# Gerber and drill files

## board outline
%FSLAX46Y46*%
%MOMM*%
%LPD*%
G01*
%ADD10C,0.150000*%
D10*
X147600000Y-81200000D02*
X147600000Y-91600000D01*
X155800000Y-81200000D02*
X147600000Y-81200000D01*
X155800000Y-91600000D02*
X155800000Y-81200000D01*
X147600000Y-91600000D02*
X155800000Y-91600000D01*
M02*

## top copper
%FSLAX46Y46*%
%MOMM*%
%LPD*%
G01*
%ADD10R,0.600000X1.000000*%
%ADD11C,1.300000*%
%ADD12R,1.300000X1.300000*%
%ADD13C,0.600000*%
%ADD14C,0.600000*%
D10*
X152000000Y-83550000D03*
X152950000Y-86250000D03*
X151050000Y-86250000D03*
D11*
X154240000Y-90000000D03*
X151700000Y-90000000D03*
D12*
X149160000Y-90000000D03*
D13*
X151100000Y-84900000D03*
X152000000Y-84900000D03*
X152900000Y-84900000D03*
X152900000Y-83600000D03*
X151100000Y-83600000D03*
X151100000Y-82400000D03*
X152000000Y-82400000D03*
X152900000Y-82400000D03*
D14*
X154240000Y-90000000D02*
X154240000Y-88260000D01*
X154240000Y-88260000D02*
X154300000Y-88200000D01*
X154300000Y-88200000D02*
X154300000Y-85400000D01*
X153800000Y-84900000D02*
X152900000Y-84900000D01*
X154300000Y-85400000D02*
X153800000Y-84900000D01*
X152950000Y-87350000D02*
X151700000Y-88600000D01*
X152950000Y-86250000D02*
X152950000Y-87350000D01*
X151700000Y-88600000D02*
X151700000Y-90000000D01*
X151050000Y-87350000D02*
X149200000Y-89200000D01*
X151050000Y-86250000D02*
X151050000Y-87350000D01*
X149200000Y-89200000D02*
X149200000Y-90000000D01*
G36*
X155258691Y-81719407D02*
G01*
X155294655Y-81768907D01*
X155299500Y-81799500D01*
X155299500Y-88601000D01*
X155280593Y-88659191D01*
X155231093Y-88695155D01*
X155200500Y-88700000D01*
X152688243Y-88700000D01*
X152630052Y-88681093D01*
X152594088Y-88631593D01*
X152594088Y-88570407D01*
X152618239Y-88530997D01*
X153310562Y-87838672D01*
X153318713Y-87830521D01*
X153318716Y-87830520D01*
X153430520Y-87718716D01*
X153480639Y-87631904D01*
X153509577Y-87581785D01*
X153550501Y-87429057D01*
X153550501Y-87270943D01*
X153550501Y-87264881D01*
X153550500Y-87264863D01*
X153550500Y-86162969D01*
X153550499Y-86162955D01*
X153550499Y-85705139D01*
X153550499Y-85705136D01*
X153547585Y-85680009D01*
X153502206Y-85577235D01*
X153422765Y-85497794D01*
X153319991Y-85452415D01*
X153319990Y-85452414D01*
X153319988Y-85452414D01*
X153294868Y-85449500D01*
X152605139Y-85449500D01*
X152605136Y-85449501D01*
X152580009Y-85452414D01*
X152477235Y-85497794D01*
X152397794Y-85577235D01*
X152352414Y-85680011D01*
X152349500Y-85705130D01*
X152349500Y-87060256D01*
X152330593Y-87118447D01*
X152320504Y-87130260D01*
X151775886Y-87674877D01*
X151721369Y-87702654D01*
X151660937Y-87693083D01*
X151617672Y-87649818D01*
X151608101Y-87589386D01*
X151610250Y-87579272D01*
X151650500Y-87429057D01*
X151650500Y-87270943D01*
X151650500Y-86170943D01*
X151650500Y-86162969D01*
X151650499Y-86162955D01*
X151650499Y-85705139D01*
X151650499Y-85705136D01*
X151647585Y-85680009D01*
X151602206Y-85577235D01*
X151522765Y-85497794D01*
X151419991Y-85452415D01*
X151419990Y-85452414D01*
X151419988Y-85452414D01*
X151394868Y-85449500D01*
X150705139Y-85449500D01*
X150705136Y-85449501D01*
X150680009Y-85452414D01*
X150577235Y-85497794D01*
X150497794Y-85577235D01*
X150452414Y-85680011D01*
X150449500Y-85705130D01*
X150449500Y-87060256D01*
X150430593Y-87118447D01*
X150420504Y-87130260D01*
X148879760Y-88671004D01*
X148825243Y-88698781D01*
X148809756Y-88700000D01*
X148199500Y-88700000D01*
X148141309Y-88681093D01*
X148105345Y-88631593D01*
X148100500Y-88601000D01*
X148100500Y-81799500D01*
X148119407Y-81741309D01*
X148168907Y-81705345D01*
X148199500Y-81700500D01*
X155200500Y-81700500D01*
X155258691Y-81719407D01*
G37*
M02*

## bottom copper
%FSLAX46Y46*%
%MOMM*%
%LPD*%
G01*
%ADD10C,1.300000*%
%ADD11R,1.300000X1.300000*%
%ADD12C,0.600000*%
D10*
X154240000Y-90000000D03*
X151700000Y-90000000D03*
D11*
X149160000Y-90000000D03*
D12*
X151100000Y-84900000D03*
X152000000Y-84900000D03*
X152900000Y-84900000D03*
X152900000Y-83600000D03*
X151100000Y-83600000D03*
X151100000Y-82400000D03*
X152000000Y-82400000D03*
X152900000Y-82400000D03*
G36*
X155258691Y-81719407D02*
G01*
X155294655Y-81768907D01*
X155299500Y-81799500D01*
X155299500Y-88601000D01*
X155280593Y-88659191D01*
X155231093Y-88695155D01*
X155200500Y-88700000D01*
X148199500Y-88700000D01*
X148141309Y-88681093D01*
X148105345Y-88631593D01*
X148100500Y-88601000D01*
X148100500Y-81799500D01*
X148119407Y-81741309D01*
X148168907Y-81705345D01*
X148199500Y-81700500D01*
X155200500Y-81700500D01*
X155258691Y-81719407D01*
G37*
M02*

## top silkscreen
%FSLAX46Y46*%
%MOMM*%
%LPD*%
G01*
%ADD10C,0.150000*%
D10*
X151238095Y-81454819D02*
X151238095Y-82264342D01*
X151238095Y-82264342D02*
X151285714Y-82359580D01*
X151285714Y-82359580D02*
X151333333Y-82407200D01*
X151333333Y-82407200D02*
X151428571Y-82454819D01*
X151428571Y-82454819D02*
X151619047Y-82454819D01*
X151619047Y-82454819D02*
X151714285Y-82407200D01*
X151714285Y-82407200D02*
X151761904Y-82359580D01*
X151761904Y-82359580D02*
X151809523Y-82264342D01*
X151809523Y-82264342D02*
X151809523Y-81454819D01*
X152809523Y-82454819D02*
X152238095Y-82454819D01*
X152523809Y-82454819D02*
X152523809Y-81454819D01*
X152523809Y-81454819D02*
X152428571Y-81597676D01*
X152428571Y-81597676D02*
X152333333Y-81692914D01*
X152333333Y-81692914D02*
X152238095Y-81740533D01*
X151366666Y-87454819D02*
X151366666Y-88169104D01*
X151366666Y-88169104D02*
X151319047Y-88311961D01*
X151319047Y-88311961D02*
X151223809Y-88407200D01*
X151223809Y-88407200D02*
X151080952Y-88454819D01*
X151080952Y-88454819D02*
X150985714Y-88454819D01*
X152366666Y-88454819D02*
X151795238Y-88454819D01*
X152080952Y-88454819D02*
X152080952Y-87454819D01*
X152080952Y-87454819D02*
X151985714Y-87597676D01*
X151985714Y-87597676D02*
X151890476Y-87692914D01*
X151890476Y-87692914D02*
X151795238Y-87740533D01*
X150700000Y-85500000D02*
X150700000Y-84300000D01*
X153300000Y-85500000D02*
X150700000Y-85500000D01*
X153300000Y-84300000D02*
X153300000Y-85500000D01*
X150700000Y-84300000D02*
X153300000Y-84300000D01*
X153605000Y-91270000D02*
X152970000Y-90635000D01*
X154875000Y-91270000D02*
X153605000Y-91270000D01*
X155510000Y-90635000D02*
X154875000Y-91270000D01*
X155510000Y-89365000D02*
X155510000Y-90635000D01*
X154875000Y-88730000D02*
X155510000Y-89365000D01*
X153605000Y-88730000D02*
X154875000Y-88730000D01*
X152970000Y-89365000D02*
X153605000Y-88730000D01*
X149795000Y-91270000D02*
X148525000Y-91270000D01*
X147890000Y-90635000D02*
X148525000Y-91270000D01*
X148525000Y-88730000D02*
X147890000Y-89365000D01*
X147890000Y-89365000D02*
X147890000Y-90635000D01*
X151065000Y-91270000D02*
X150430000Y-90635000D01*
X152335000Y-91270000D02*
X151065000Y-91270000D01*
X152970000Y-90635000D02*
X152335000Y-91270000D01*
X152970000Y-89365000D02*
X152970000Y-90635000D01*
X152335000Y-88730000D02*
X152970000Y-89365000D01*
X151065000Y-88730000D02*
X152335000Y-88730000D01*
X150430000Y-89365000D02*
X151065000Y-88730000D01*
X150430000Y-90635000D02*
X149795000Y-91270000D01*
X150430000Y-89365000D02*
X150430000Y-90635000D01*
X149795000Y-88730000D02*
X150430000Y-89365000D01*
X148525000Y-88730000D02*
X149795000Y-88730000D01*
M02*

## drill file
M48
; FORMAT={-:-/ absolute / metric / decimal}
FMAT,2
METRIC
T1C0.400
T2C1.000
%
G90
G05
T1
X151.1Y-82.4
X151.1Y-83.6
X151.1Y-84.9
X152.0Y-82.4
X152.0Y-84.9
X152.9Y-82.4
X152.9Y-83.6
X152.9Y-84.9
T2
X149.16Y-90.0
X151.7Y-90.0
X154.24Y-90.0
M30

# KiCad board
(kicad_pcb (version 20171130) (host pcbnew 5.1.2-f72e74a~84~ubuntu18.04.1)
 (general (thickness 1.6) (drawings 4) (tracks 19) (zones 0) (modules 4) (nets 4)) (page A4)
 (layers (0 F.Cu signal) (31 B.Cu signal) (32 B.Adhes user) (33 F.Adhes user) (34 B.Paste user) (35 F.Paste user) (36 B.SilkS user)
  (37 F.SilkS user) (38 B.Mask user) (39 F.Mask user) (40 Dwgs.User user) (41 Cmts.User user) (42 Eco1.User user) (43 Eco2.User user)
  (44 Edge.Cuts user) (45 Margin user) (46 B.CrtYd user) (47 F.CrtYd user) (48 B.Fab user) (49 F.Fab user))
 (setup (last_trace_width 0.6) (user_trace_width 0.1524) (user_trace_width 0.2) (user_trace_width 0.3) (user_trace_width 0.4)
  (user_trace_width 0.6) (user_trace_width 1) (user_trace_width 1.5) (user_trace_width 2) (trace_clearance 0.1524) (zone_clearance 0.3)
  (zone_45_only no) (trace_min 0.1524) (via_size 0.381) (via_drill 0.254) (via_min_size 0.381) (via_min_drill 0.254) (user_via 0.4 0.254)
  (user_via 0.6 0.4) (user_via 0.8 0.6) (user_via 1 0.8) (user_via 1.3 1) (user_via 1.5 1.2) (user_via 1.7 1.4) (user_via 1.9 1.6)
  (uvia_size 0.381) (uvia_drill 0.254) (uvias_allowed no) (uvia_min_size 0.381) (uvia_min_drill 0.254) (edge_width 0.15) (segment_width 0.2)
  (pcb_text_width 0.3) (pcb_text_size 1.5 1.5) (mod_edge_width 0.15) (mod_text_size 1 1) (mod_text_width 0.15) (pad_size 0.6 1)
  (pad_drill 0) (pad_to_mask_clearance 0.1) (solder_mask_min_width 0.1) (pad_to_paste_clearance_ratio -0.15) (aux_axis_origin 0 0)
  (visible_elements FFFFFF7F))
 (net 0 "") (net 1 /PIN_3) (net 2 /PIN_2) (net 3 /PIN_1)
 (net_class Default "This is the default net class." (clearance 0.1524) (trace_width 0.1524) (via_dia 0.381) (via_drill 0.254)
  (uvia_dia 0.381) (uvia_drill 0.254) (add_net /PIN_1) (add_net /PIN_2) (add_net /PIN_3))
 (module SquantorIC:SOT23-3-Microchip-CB (layer F.Cu) (at 152 84.9)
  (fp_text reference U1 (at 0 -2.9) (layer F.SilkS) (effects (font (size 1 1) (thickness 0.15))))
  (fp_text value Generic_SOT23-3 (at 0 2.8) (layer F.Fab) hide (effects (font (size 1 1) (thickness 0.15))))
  (fp_line (start -1.3 0.6) (end -1.3 -0.6) (layer F.SilkS) (width 0.15))
  (fp_line (start 1.3 0.6) (end -1.3 0.6) (layer F.SilkS) (width 0.15))
  (fp_line (start 1.3 -0.6) (end 1.3 0.6) (layer F.SilkS) (width 0.15))
  (fp_line (start -1.3 -0.6) (end 1.3 -0.6) (layer F.SilkS) (width 0.15))
  (pad 3 smd rect (at 0 -1.35) (size 0.6 1) (layers F.Cu F.Paste F.Mask) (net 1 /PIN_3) (zone_connect 2))
  (pad 2 smd rect (at 0.95 1.35) (size 0.6 1) (layers F.Cu F.Paste F.Mask) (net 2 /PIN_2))
  (pad 1 smd rect (at -0.95 1.35) (size 0.6 1) (layers F.Cu F.Paste F.Mask) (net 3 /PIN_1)))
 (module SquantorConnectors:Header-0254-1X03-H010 (layer F.Cu) (at 151.7 90)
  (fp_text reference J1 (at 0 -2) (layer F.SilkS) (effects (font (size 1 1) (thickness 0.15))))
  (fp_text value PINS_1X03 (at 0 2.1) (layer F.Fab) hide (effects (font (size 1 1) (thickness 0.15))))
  (fp_line (start 1.905 1.27) (end 1.27 0.635) (layer F.SilkS) (width 0.15))
  (fp_line (start 3.175 1.27) (end 1.905 1.27) (layer F.SilkS) (width 0.15))
  (fp_line (start 3.81 0.635) (end 3.175 1.27) (layer F.SilkS) (width 0.15))
  (fp_line (start 3.81 -0.635) (end 3.81 0.635) (layer F.SilkS) (width 0.15))
  (fp_line (start 3.175 -1.27) (end 3.81 -0.635) (layer F.SilkS) (width 0.15))
  (fp_line (start 1.905 -1.27) (end 3.175 -1.27) (layer F.SilkS) (width 0.15))
  (fp_line (start 1.27 -0.635) (end 1.905 -1.27) (layer F.SilkS) (width 0.15))
  (fp_line (start -1.905 1.27) (end -3.175 1.27) (layer F.SilkS) (width 0.15))
  (fp_line (start -3.81 0.635) (end -3.175 1.27) (layer F.SilkS) (width 0.15))
  (fp_line (start -3.175 -1.27) (end -3.81 -0.635) (layer F.SilkS) (width 0.15))
  (fp_line (start -3.81 -0.635) (end -3.81 0.635) (layer F.SilkS) (width 0.15))
  (fp_line (start -0.635 1.27) (end -1.27 0.635) (layer F.SilkS) (width 0.15))
  (fp_line (start 0.635 1.27) (end -0.635 1.27) (layer F.SilkS) (width 0.15))
  (fp_line (start 1.27 0.635) (end 0.635 1.27) (layer F.SilkS) (width 0.15))
  (fp_line (start 1.27 -0.635) (end 1.27 0.635) (layer F.SilkS) (width 0.15))
  (fp_line (start 0.635 -1.27) (end 1.27 -0.635) (layer F.SilkS) (width 0.15))
  (fp_line (start -0.635 -1.27) (end 0.635 -1.27) (layer F.SilkS) (width 0.15))
  (fp_line (start -1.27 -0.635) (end -0.635 -1.27) (layer F.SilkS) (width 0.15))
  (fp_line (start -1.27 0.635) (end -1.905 1.27) (layer F.SilkS) (width 0.15))
  (fp_line (start -1.27 -0.635) (end -1.27 0.635) (layer F.SilkS) (width 0.15))
  (fp_line (start -1.905 -1.27) (end -1.27 -0.635) (layer F.SilkS) (width 0.15))
  (fp_line (start -3.175 -1.27) (end -1.905 -1.27) (layer F.SilkS) (width 0.15))
  (pad 3 thru_hole circle (at 2.54 0 180) (size 1.3 1.3) (drill 1) (layers *.Cu *.Mask) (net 1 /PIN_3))
  (pad 2 thru_hole circle (at 0 0 180) (size 1.3 1.3) (drill 1) (layers *.Cu *.Mask) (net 2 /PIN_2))
  (pad 1 thru_hole rect (at -2.54 0 180) (size 1.3 1.3) (drill 1) (layers *.Cu *.Mask) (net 3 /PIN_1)))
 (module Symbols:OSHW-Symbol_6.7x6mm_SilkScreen (layer B.Cu) (at 152 84.6 180)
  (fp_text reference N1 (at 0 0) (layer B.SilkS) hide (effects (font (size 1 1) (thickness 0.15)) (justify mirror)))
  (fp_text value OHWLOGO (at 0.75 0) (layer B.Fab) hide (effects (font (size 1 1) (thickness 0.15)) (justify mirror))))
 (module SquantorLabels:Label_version (layer B.Cu) (at 152 88.2)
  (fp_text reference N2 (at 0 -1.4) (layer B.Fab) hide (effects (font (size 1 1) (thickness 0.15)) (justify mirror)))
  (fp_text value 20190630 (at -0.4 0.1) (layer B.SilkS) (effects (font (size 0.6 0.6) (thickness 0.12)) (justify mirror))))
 (gr_line (start 147.6 81.2) (end 147.6 91.6) (layer Edge.Cuts) (width 0.15))
 (gr_line (start 155.8 81.2) (end 147.6 81.2) (layer Edge.Cuts) (width 0.15))
 (gr_line (start 155.8 91.6) (end 155.8 81.2) (layer Edge.Cuts) (width 0.15))
 (gr_line (start 147.6 91.6) (end 155.8 91.6) (layer Edge.Cuts) (width 0.15))
 (via (at 151.1 84.9) (size 0.6) (drill 0.4) (layers F.Cu B.Cu) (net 1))
 (via (at 152 84.9) (size 0.6) (drill 0.4) (layers F.Cu B.Cu) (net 1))
 (via (at 152.9 84.9) (size 0.6) (drill 0.4) (layers F.Cu B.Cu) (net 1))
 (via (at 152.9 83.6) (size 0.6) (drill 0.4) (layers F.Cu B.Cu) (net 1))
 (via (at 151.1 83.6) (size 0.6) (drill 0.4) (layers F.Cu B.Cu) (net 1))
 (via (at 151.1 82.4) (size 0.6) (drill 0.4) (layers F.Cu B.Cu) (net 1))
 (via (at 152 82.4) (size 0.6) (drill 0.4) (layers F.Cu B.Cu) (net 1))
 (via (at 152.9 82.4) (size 0.6) (drill 0.4) (layers F.Cu B.Cu) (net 1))
 (segment (start 154.24 90) (end 154.24 88.26) (width 0.6) (layer F.Cu) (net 1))
 (segment (start 154.24 88.26) (end 154.3 88.2) (width 0.6) (layer F.Cu) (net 1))
 (segment (start 154.3 88.2) (end 154.3 85.4) (width 0.6) (layer F.Cu) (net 1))
 (segment (start 153.8 84.9) (end 152.9 84.9) (width 0.6) (layer F.Cu) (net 1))
 (segment (start 154.3 85.4) (end 153.8 84.9) (width 0.6) (layer F.Cu) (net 1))
 (segment (start 152.95 87.35) (end 151.7 88.6) (width 0.6) (layer F.Cu) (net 2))
 (segment (start 152.95 86.25) (end 152.95 87.35) (width 0.6) (layer F.Cu) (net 2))
 (segment (start 151.7 88.6) (end 151.7 90) (width 0.6) (layer F.Cu) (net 2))
 (segment (start 151.05 87.35) (end 149.2 89.2) (width 0.6) (layer F.Cu) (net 3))
 (segment (start 151.05 86.25) (end 151.05 87.35) (width 0.6) (layer F.Cu) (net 3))
 (segment (start 149.2 89.2) (end 149.2 90) (width 0.6) (layer F.Cu) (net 3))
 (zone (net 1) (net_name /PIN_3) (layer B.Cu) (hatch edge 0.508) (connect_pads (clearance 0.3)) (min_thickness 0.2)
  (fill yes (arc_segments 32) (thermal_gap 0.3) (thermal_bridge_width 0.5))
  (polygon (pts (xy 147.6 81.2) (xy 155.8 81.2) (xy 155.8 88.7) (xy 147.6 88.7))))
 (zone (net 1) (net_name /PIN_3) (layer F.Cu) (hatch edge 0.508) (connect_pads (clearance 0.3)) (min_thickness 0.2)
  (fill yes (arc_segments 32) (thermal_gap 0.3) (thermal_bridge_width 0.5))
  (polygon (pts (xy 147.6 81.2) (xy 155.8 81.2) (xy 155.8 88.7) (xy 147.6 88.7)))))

